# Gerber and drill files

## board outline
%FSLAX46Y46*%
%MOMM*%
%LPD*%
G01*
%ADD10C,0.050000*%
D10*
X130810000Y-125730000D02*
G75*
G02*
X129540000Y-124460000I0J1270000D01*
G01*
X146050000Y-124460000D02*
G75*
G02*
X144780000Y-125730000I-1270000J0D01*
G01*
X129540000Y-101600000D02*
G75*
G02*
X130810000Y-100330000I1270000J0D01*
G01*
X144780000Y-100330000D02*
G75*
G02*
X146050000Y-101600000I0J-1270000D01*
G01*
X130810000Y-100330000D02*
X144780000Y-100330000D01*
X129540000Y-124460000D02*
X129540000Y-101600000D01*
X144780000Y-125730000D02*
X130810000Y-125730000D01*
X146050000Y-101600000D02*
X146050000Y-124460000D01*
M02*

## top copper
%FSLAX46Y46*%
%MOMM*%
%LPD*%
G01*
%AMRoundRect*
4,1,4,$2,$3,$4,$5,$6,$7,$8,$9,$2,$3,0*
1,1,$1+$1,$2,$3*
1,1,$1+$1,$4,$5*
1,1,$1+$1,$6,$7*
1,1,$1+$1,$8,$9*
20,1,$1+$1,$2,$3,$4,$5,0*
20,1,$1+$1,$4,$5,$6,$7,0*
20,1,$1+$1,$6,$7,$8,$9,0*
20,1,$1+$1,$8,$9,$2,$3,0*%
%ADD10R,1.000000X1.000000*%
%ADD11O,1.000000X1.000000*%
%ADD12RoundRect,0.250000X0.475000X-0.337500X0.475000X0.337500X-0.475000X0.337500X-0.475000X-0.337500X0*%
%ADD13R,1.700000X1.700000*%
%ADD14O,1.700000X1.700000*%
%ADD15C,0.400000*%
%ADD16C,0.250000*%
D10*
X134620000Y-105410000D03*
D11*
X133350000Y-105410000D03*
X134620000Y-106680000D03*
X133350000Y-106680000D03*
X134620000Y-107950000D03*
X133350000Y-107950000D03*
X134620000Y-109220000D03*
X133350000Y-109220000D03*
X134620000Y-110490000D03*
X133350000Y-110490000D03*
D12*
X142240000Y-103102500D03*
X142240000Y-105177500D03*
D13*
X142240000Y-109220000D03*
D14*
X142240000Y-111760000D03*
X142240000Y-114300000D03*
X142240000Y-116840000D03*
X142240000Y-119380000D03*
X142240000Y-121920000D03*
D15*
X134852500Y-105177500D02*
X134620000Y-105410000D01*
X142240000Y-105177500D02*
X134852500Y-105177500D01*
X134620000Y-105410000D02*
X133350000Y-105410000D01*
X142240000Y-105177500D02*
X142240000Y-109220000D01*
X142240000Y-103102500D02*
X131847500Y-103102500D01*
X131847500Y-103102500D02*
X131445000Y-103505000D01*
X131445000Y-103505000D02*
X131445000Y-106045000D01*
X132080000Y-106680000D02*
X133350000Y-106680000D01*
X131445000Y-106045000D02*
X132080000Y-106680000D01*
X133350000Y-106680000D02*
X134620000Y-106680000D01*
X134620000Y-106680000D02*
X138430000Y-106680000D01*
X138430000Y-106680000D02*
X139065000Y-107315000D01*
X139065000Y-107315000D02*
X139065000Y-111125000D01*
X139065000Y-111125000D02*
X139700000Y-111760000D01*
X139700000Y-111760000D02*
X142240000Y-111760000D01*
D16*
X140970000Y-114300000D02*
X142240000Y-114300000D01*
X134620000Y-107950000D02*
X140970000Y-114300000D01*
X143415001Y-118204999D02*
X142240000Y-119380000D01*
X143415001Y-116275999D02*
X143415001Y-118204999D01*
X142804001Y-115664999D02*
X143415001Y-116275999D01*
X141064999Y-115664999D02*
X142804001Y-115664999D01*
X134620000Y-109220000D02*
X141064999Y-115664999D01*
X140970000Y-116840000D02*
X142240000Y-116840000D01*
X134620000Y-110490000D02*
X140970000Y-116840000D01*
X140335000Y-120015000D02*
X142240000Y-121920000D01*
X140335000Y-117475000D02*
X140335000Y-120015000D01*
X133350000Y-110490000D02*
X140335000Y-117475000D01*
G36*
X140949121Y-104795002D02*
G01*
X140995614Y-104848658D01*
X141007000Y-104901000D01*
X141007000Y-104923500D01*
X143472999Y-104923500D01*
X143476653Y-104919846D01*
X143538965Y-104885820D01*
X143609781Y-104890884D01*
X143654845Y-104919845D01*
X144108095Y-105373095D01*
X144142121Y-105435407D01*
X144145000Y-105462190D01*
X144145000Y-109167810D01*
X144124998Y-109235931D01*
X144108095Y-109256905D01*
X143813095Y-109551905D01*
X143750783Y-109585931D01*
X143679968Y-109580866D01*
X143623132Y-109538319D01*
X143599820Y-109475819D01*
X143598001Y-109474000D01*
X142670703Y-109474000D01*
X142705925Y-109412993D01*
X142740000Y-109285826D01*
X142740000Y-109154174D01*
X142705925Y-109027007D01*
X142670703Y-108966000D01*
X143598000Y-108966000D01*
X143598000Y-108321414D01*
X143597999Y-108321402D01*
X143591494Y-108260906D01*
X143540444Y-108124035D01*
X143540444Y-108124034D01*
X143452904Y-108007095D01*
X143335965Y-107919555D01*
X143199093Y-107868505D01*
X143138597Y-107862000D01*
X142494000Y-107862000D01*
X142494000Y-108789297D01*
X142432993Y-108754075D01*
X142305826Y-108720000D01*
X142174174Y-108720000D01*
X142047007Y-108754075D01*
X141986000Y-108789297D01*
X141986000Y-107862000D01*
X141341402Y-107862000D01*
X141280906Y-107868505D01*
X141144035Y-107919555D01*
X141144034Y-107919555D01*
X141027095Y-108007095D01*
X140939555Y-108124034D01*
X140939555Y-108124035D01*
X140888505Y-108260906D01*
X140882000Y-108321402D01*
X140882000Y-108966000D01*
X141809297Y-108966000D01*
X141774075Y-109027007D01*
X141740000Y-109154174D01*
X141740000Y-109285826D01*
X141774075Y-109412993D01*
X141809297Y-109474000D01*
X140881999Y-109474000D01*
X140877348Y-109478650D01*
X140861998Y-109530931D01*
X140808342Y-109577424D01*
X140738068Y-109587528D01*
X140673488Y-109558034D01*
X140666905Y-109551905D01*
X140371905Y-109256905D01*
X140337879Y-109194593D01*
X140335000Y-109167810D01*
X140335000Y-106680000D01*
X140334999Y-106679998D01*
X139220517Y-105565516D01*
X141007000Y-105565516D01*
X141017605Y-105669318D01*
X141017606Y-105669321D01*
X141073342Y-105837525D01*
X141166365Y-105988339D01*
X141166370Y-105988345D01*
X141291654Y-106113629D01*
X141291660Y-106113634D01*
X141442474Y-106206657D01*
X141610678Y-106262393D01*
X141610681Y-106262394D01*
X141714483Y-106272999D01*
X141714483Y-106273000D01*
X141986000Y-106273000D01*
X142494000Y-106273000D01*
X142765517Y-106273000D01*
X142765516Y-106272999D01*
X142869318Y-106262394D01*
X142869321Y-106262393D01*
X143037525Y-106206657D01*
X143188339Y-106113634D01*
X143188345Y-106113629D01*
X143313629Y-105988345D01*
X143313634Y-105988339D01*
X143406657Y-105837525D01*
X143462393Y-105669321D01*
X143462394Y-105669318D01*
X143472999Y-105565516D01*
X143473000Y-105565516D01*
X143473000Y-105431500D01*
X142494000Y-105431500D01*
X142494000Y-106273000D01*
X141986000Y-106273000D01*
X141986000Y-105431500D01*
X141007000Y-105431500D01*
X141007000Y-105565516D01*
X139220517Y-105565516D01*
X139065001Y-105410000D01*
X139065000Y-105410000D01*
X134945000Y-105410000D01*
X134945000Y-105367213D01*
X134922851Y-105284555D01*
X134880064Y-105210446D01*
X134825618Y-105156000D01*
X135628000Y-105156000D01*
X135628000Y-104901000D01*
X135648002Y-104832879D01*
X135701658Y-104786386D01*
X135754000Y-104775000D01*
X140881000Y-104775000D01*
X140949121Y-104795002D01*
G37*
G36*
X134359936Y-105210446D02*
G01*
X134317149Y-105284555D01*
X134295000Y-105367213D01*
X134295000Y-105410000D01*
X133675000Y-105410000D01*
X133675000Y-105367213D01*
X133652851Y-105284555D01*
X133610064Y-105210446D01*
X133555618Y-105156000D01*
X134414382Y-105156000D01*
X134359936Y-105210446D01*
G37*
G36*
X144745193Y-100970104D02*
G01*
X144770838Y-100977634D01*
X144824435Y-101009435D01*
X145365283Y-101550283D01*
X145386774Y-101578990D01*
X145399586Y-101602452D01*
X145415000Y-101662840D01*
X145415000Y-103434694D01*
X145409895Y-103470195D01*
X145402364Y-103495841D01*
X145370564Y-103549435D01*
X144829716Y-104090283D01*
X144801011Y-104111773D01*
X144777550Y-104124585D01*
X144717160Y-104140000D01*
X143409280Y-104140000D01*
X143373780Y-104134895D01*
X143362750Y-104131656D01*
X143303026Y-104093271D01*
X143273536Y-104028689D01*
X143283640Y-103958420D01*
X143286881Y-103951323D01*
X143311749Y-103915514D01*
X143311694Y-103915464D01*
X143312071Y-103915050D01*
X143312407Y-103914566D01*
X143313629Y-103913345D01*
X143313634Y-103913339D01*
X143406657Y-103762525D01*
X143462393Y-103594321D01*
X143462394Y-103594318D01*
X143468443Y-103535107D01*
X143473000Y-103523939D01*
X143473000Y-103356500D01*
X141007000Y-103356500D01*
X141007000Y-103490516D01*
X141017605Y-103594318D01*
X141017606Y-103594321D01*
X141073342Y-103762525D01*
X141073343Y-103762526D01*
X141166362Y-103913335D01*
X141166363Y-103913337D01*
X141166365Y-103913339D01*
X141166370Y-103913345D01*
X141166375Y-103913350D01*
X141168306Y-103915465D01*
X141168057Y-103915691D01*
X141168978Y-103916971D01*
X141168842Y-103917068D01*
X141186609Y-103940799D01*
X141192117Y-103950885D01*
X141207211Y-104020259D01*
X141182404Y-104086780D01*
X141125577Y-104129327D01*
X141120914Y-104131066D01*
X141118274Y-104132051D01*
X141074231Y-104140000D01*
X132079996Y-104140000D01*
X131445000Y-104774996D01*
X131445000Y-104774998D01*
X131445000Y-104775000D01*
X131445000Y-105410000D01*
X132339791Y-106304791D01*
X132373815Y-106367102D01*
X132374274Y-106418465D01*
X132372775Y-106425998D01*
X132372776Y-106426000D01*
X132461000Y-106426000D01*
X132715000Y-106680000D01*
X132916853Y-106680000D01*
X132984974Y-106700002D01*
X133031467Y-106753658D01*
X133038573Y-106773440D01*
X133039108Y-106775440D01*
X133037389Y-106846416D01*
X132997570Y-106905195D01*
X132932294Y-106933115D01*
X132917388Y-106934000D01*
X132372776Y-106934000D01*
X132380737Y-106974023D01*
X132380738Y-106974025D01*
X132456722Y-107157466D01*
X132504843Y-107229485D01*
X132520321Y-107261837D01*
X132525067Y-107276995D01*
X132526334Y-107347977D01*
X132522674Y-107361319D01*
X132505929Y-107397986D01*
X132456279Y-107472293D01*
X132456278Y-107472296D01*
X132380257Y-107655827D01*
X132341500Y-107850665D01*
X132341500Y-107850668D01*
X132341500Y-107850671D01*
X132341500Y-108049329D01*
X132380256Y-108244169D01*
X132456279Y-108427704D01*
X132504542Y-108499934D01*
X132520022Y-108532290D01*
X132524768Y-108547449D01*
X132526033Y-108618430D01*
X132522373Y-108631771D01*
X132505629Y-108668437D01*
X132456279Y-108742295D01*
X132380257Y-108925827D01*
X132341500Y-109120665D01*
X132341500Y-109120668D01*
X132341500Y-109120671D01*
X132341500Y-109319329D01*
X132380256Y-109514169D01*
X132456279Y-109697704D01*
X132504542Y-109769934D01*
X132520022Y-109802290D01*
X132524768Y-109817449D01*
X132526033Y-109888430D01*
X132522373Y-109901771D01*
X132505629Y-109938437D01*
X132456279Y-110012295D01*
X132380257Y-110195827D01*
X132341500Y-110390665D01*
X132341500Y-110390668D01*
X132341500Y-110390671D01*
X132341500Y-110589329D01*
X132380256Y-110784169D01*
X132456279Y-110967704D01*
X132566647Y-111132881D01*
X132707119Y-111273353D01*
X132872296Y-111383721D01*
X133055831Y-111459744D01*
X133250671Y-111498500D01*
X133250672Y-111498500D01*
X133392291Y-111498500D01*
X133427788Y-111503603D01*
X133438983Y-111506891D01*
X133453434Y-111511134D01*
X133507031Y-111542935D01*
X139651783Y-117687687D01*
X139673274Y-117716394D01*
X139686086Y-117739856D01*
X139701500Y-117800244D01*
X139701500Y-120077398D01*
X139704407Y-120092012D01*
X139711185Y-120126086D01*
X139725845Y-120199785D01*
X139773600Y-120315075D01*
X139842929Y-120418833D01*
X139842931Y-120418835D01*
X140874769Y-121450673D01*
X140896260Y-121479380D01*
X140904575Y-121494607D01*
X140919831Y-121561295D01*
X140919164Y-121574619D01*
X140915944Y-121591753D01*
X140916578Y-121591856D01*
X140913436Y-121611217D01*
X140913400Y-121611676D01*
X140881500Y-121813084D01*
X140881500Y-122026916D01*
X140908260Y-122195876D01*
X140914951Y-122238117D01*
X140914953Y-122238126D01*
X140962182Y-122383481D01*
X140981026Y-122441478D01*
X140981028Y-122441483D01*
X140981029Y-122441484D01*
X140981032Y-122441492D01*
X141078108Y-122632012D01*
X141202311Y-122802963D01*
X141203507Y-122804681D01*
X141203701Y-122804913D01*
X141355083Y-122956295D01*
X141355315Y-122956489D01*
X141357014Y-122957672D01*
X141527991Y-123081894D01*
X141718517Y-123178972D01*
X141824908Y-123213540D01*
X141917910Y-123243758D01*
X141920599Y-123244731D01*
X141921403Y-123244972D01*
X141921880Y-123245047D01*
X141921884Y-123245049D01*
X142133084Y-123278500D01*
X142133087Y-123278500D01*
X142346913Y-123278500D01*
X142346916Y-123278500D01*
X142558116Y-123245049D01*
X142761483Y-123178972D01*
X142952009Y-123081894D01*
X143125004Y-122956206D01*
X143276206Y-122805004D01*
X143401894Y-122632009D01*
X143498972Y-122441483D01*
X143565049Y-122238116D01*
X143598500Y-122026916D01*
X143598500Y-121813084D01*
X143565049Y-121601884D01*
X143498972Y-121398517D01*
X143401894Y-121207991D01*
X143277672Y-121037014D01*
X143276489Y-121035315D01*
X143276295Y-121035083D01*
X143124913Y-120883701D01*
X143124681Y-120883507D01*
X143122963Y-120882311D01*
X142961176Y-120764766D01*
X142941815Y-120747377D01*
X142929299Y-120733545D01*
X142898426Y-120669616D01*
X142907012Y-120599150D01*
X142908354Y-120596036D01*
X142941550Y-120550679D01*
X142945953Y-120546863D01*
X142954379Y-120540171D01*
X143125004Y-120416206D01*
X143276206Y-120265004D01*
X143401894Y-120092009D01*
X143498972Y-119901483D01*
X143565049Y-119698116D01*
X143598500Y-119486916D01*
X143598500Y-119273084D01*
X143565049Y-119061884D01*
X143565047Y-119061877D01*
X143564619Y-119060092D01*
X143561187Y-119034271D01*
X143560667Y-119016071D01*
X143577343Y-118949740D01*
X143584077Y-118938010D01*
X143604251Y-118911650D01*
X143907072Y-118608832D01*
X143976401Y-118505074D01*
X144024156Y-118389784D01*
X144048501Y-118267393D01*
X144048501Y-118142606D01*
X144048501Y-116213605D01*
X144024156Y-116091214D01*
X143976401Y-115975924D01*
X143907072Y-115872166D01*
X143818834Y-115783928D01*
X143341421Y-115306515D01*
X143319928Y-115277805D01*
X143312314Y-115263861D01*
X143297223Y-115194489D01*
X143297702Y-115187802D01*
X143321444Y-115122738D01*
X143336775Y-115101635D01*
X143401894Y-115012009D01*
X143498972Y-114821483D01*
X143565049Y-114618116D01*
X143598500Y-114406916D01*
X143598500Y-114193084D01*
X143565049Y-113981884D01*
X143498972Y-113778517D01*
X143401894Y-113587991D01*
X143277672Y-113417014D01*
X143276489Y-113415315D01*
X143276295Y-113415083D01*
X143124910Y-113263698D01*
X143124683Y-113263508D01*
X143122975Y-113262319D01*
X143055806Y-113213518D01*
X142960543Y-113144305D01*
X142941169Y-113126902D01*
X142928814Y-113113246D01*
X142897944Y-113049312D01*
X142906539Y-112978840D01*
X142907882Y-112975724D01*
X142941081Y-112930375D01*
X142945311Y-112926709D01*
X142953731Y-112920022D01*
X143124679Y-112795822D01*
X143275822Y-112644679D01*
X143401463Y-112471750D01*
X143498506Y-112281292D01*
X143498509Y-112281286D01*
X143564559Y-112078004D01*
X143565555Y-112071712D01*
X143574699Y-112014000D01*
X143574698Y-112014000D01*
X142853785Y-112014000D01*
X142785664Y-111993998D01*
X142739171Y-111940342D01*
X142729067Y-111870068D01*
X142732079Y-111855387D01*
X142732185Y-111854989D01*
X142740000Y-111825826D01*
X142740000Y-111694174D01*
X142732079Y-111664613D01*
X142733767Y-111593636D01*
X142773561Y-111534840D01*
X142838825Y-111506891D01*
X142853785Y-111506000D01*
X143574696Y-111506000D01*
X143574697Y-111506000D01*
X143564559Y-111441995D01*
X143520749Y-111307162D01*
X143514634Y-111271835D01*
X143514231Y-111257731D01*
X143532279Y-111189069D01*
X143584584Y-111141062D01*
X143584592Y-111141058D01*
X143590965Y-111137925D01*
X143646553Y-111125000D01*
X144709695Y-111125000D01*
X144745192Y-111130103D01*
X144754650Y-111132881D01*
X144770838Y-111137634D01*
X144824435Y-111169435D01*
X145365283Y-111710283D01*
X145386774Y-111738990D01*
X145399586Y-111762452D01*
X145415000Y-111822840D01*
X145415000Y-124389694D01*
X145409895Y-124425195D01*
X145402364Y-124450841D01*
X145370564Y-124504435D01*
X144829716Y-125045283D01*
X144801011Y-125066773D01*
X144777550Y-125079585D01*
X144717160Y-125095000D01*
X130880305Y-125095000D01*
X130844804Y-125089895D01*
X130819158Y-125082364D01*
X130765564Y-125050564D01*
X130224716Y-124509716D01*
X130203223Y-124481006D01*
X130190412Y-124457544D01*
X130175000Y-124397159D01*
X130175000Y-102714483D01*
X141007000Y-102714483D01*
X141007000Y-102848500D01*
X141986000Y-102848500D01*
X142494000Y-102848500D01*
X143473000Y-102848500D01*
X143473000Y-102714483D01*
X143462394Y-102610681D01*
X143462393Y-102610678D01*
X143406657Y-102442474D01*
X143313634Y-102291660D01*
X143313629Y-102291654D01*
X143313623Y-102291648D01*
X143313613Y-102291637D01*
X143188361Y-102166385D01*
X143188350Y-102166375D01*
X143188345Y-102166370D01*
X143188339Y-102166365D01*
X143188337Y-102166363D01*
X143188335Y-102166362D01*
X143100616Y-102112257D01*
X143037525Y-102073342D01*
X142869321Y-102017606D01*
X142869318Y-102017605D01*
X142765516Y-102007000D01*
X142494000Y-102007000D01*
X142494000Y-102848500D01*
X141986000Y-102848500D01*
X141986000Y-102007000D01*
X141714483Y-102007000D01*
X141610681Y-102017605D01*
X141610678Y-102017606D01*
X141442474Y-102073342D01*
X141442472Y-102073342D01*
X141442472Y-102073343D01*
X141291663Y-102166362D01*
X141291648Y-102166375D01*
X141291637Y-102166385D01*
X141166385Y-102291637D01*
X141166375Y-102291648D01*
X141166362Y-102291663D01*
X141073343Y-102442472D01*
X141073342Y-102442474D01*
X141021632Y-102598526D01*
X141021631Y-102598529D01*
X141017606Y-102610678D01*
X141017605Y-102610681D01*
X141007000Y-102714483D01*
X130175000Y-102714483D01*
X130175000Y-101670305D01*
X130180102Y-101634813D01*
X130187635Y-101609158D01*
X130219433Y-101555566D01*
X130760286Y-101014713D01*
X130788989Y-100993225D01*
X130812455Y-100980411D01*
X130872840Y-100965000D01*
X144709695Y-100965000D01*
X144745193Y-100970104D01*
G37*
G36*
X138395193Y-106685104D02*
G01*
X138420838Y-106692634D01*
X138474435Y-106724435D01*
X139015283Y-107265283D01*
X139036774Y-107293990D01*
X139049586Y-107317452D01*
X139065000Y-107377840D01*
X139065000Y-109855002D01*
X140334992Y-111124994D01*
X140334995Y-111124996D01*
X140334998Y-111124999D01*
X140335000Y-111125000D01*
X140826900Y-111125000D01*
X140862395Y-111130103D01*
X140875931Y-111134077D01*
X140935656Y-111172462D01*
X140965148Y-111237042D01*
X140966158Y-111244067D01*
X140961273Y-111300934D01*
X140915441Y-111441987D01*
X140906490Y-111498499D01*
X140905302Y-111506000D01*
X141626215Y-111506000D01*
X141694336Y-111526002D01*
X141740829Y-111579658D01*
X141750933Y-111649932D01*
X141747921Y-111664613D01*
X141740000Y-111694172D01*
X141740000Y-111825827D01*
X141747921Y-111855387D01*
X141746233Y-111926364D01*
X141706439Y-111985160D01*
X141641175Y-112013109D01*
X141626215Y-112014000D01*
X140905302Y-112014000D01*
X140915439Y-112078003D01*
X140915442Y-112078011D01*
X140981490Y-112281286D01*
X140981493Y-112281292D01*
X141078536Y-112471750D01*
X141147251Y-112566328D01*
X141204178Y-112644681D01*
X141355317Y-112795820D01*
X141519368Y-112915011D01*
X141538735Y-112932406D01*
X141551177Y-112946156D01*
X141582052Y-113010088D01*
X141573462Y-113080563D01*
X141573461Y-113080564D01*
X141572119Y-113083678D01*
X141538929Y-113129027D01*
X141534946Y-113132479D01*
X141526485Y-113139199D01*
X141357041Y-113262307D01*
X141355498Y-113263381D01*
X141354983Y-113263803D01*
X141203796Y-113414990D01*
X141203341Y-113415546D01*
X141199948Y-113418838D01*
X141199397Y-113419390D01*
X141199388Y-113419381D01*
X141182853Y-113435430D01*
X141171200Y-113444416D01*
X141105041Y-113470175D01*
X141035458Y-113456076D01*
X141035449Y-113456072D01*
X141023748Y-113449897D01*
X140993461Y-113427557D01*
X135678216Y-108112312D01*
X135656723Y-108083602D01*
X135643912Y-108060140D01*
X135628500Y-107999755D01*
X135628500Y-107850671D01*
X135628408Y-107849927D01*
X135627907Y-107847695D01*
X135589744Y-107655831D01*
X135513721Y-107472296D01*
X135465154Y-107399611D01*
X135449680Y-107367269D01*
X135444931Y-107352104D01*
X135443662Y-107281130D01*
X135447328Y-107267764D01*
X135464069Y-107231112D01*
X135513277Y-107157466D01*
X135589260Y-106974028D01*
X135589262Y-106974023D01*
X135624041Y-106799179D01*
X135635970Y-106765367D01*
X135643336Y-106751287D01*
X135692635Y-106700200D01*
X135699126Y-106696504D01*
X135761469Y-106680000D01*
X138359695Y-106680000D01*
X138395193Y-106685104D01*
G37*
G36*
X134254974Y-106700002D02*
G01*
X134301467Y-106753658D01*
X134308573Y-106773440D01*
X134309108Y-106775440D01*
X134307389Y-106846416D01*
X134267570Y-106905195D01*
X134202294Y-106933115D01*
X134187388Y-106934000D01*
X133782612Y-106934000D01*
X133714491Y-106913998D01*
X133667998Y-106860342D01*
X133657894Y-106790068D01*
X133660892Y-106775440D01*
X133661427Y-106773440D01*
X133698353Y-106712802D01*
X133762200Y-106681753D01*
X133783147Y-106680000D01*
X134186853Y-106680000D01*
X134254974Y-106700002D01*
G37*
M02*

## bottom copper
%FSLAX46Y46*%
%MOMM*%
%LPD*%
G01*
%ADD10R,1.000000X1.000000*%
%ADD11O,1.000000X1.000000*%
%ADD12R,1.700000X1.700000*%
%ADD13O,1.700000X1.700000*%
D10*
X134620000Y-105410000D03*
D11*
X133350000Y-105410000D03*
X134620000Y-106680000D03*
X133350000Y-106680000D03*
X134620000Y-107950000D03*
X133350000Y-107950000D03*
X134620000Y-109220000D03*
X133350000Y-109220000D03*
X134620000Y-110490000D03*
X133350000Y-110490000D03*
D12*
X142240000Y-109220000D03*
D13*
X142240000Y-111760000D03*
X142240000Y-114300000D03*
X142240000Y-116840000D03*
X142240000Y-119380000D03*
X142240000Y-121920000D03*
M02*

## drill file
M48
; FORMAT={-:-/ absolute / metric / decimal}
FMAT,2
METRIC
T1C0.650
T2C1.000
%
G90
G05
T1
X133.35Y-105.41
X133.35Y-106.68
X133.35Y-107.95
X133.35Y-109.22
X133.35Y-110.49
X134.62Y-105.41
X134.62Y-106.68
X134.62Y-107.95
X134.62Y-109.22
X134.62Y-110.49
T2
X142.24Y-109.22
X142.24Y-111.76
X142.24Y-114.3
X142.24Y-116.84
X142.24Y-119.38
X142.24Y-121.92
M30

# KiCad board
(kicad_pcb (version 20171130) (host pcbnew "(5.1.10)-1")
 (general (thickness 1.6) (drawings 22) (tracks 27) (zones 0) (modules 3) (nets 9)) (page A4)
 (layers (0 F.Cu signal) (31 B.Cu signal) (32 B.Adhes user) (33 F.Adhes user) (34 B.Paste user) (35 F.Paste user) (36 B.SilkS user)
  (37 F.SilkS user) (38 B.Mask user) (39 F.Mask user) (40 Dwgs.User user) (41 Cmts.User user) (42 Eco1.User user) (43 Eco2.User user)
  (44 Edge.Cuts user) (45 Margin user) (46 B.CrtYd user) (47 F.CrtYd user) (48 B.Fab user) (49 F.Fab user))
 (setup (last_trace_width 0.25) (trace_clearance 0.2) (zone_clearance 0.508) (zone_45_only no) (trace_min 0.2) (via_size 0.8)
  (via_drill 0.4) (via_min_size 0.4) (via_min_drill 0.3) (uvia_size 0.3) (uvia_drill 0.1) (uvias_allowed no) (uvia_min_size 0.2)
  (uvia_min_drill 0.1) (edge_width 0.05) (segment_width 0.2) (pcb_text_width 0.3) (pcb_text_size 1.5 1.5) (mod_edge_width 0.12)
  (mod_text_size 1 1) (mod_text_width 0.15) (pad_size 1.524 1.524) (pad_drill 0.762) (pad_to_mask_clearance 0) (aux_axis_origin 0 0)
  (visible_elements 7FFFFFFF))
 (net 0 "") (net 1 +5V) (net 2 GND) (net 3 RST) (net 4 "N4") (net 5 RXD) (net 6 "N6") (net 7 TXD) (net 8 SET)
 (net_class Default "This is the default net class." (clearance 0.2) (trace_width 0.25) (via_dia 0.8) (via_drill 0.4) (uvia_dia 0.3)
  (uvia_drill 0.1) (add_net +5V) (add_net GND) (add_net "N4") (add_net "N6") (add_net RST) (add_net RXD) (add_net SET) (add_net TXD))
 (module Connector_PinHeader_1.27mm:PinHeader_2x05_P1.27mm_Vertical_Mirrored (layer F.Cu) (at 133.35 105.41)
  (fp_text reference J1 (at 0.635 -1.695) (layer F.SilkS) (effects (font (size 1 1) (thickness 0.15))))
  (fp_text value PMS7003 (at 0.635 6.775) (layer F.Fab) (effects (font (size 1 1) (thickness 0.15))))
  (pad 1 thru_hole rect (at 1.27 0) (size 1 1) (drill 0.65) (layers *.Cu *.Mask) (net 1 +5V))
  (pad 2 thru_hole oval (at 0 0) (size 1 1) (drill 0.65) (layers *.Cu *.Mask) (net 1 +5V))
  (pad 3 thru_hole oval (at 1.27 1.27) (size 1 1) (drill 0.65) (layers *.Cu *.Mask) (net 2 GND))
  (pad 4 thru_hole oval (at 0 1.27) (size 1 1) (drill 0.65) (layers *.Cu *.Mask) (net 2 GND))
  (pad 5 thru_hole oval (at 1.27 2.54) (size 1 1) (drill 0.65) (layers *.Cu *.Mask) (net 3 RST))
  (pad 6 thru_hole oval (at 0 2.54) (size 1 1) (drill 0.65) (layers *.Cu *.Mask) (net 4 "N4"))
  (pad 7 thru_hole oval (at 1.27 3.81) (size 1 1) (drill 0.65) (layers *.Cu *.Mask) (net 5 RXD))
  (pad 8 thru_hole oval (at 0 3.81) (size 1 1) (drill 0.65) (layers *.Cu *.Mask) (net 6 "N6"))
  (pad 9 thru_hole oval (at 1.27 5.08) (size 1 1) (drill 0.65) (layers *.Cu *.Mask) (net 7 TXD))
  (pad 10 thru_hole oval (at 0 5.08) (size 1 1) (drill 0.65) (layers *.Cu *.Mask) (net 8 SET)))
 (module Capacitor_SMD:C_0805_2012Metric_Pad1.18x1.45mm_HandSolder (layer F.Cu) (at 142.24 104.14 90)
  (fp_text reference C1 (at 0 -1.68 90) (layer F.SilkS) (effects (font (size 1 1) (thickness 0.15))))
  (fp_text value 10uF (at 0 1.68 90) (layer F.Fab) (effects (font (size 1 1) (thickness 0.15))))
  (pad 2 smd roundrect (at 1.0375 0 90) (size 1.175 1.45) (layers F.Cu F.Paste F.Mask) (roundrect_rratio 0.212766) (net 2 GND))
  (pad 1 smd roundrect (at -1.0375 0 90) (size 1.175 1.45) (layers F.Cu F.Paste F.Mask) (roundrect_rratio 0.212766) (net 1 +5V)))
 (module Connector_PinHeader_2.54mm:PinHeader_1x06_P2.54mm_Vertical (layer F.Cu) (at 142.24 109.22)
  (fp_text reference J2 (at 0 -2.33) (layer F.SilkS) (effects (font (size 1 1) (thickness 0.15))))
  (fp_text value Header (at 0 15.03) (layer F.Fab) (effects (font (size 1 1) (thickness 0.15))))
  (pad 1 thru_hole rect (at 0 0) (size 1.7 1.7) (drill 1) (layers *.Cu *.Mask) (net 1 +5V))
  (pad 2 thru_hole oval (at 0 2.54) (size 1.7 1.7) (drill 1) (layers *.Cu *.Mask) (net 2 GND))
  (pad 3 thru_hole oval (at 0 5.08) (size 1.7 1.7) (drill 1) (layers *.Cu *.Mask) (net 3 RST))
  (pad 4 thru_hole oval (at 0 7.62) (size 1.7 1.7) (drill 1) (layers *.Cu *.Mask) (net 7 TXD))
  (pad 5 thru_hole oval (at 0 10.16) (size 1.7 1.7) (drill 1) (layers *.Cu *.Mask) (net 5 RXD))
  (pad 6 thru_hole oval (at 0 12.7) (size 1.7 1.7) (drill 1) (layers *.Cu *.Mask) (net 8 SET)))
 (gr_arc (start 130.81 124.46) (end 129.54 124.46) (angle -90) (layer Edge.Cuts) (width 0.05))
 (gr_arc (start 144.78 124.46) (end 144.78 125.73) (angle -90) (layer Edge.Cuts) (width 0.05))
 (gr_arc (start 130.81 101.6) (end 130.81 100.33) (angle -90) (layer Edge.Cuts) (width 0.05))
 (gr_arc (start 144.78 101.6) (end 146.05 101.6) (angle -90) (layer Edge.Cuts) (width 0.05))
 (gr_line (start 130.81 100.33) (end 144.78 100.33) (layer Edge.Cuts) (width 0.05))
 (gr_line (start 129.54 124.46) (end 129.54 101.6) (layer Edge.Cuts) (width 0.05))
 (gr_line (start 144.78 125.73) (end 130.81 125.73) (layer Edge.Cuts) (width 0.05))
 (gr_line (start 146.05 101.6) (end 146.05 124.46) (layer Edge.Cuts) (width 0.05))
 (segment (start 134.8525 105.1775) (end 134.62 105.41) (width 0.4) (layer F.Cu) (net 1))
 (segment (start 142.24 105.1775) (end 134.8525 105.1775) (width 0.4) (layer F.Cu) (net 1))
 (segment (start 134.62 105.41) (end 133.35 105.41) (width 0.4) (layer F.Cu) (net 1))
 (segment (start 142.24 105.1775) (end 142.24 109.22) (width 0.4) (layer F.Cu) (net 1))
 (segment (start 142.24 103.1025) (end 131.8475 103.1025) (width 0.4) (layer F.Cu) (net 2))
 (segment (start 131.8475 103.1025) (end 131.445 103.505) (width 0.4) (layer F.Cu) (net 2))
 (segment (start 131.445 103.505) (end 131.445 106.045) (width 0.4) (layer F.Cu) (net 2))
 (segment (start 132.08 106.68) (end 133.35 106.68) (width 0.4) (layer F.Cu) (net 2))
 (segment (start 131.445 106.045) (end 132.08 106.68) (width 0.4) (layer F.Cu) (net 2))
 (segment (start 133.35 106.68) (end 134.62 106.68) (width 0.4) (layer F.Cu) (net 2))
 (segment (start 134.62 106.68) (end 138.43 106.68) (width 0.4) (layer F.Cu) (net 2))
 (segment (start 138.43 106.68) (end 139.065 107.315) (width 0.4) (layer F.Cu) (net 2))
 (segment (start 139.065 107.315) (end 139.065 111.125) (width 0.4) (layer F.Cu) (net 2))
 (segment (start 139.065 111.125) (end 139.7 111.76) (width 0.4) (layer F.Cu) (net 2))
 (segment (start 139.7 111.76) (end 142.24 111.76) (width 0.4) (layer F.Cu) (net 2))
 (segment (start 140.97 114.3) (end 142.24 114.3) (width 0.25) (layer F.Cu) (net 3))
 (segment (start 134.62 107.95) (end 140.97 114.3) (width 0.25) (layer F.Cu) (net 3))
 (segment (start 143.415001 118.204999) (end 142.24 119.38) (width 0.25) (layer F.Cu) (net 5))
 (segment (start 143.415001 116.275999) (end 143.415001 118.204999) (width 0.25) (layer F.Cu) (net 5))
 (segment (start 142.804001 115.664999) (end 143.415001 116.275999) (width 0.25) (layer F.Cu) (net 5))
 (segment (start 141.064999 115.664999) (end 142.804001 115.664999) (width 0.25) (layer F.Cu) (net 5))
 (segment (start 134.62 109.22) (end 141.064999 115.664999) (width 0.25) (layer F.Cu) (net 5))
 (segment (start 140.97 116.84) (end 142.24 116.84) (width 0.25) (layer F.Cu) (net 7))
 (segment (start 134.62 110.49) (end 140.97 116.84) (width 0.25) (layer F.Cu) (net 7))
 (segment (start 140.335 120.015) (end 142.24 121.92) (width 0.25) (layer F.Cu) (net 8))
 (segment (start 140.335 117.475) (end 140.335 120.015) (width 0.25) (layer F.Cu) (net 8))
 (segment (start 133.35 110.49) (end 140.335 117.475) (width 0.25) (layer F.Cu) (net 8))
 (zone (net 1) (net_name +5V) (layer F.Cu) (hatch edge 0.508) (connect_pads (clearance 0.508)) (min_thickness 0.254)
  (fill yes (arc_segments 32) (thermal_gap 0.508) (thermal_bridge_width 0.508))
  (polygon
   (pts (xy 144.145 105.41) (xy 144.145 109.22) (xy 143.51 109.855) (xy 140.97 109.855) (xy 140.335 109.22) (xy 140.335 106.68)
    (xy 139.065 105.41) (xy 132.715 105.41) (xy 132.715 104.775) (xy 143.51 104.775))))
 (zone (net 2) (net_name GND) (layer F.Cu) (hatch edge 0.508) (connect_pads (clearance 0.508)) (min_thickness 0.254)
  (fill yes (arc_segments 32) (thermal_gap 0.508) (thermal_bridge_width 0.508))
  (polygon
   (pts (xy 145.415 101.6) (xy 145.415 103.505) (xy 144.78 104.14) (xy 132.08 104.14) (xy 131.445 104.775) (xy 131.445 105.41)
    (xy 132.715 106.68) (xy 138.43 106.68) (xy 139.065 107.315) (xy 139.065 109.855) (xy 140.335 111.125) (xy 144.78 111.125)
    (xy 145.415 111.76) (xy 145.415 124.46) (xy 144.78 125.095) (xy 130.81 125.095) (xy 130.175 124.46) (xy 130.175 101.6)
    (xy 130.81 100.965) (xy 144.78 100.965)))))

